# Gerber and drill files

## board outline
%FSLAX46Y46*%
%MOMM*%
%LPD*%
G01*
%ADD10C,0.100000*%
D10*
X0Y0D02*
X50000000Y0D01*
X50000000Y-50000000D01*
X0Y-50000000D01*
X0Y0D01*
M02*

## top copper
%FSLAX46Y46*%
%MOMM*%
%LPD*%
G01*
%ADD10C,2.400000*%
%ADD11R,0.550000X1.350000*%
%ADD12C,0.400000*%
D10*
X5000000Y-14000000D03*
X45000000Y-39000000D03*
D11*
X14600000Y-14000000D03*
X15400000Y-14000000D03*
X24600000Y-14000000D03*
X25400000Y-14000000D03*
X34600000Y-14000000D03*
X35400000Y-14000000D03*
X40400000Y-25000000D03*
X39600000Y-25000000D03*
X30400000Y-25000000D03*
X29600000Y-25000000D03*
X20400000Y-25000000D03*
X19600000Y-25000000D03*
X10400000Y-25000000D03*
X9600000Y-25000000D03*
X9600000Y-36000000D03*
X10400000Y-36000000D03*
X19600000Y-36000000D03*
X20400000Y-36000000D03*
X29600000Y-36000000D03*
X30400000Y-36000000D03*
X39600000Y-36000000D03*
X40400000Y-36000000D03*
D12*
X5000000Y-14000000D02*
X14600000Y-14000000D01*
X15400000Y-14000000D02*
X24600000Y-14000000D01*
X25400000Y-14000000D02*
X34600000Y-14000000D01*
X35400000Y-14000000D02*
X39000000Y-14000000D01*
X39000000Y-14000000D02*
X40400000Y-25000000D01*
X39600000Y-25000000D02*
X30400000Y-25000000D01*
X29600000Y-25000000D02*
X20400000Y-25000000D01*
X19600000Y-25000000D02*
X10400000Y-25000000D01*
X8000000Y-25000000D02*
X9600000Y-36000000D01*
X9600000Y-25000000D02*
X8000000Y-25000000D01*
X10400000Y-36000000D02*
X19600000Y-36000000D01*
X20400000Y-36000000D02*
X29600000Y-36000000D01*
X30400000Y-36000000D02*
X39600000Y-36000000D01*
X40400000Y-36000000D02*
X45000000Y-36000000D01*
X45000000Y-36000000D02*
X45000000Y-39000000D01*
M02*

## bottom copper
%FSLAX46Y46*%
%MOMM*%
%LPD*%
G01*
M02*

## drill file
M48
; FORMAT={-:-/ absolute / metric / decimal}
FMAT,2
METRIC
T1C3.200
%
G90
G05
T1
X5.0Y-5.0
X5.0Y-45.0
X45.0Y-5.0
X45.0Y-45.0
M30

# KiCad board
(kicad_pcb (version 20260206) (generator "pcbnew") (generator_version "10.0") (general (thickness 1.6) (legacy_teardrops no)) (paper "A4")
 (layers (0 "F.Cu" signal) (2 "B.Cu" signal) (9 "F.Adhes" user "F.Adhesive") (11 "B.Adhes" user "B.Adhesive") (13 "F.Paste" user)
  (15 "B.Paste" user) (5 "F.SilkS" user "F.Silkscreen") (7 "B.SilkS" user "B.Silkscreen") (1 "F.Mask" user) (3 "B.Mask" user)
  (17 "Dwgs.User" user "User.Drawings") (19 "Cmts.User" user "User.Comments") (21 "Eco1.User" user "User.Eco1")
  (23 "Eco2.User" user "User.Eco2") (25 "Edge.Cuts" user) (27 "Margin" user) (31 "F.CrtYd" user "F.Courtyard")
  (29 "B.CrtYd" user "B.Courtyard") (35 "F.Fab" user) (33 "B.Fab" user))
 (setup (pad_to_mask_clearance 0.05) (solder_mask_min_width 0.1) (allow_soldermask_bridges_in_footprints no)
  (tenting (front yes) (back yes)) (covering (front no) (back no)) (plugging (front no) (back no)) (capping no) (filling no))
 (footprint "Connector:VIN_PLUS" (layer "F.Cu") (at 5 14)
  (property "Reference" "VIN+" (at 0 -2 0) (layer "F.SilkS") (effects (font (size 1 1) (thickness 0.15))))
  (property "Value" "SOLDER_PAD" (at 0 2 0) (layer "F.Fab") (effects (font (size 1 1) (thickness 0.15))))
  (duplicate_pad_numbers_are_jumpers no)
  (pad "1" smd circle (at 0 0) (size 2.4 2.4) (layers "F.Cu" "F.Mask" "F.Paste") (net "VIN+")))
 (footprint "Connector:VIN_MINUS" (layer "F.Cu") (at 45 39)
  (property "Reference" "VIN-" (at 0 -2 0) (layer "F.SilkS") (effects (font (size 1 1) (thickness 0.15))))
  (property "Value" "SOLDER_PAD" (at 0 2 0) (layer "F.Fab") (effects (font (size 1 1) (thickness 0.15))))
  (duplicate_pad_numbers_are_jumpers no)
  (pad "1" smd circle (at 0 0) (size 2.4 2.4) (layers "F.Cu" "F.Mask" "F.Paste") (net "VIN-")))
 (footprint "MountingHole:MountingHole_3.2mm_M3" (layer "F.Cu") (at 5 5)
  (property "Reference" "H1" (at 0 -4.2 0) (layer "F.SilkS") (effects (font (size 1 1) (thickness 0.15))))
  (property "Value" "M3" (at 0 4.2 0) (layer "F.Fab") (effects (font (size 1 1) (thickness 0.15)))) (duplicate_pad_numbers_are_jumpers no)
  (pad "" np_thru_hole circle (at 0 0) (size 3.2 3.2) (drill 3.2) (layers "*.Cu" "*.Mask")))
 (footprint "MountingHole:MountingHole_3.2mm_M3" (layer "F.Cu") (at 45 5)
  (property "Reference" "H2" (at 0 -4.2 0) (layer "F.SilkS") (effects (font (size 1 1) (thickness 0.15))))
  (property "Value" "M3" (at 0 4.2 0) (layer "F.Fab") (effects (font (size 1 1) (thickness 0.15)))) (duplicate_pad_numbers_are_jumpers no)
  (pad "" np_thru_hole circle (at 0 0) (size 3.2 3.2) (drill 3.2) (layers "*.Cu" "*.Mask")))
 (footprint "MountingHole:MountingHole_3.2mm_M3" (layer "F.Cu") (at 5 45)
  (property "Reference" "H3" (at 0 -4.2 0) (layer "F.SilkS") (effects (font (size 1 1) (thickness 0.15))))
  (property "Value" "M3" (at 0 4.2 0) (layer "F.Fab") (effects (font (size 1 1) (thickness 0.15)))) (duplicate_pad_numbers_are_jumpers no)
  (pad "" np_thru_hole circle (at 0 0) (size 3.2 3.2) (drill 3.2) (layers "*.Cu" "*.Mask")))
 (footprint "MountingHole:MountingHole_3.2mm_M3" (layer "F.Cu") (at 45 45)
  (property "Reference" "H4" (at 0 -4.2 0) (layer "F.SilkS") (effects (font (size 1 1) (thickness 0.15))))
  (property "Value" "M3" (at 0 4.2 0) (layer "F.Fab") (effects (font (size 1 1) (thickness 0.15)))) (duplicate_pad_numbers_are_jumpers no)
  (pad "" np_thru_hole circle (at 0 0) (size 3.2 3.2) (drill 3.2) (layers "*.Cu" "*.Mask")))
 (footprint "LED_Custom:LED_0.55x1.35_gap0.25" (layer "F.Cu") (at 15 14)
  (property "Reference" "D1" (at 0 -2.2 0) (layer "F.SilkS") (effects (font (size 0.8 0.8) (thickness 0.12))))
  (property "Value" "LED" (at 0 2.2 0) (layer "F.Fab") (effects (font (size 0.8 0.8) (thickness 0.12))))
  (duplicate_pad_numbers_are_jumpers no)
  (pad "A" smd rect (at -0.4 0) (size 0.55 1.35) (layers "F.Cu" "F.Mask" "F.Paste") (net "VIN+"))
  (pad "K" smd rect (at 0.4 0) (size 0.55 1.35) (layers "F.Cu" "F.Mask" "F.Paste") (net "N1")))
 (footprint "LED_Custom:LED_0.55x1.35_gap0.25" (layer "F.Cu") (at 25 14)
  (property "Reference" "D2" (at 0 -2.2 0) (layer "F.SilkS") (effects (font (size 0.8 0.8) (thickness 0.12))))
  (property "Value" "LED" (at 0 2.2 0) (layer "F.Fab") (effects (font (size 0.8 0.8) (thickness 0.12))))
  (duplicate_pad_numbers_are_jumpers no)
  (pad "A" smd rect (at -0.4 0) (size 0.55 1.35) (layers "F.Cu" "F.Mask" "F.Paste") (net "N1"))
  (pad "K" smd rect (at 0.4 0) (size 0.55 1.35) (layers "F.Cu" "F.Mask" "F.Paste") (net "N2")))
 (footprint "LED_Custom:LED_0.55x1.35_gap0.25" (layer "F.Cu") (at 35 14)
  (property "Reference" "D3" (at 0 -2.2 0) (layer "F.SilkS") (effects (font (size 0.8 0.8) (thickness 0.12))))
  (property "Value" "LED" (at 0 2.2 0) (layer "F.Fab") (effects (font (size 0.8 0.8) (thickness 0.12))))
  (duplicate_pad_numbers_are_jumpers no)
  (pad "A" smd rect (at -0.4 0) (size 0.55 1.35) (layers "F.Cu" "F.Mask" "F.Paste") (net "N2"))
  (pad "K" smd rect (at 0.4 0) (size 0.55 1.35) (layers "F.Cu" "F.Mask" "F.Paste") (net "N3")))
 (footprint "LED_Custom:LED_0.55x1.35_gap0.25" (layer "F.Cu") (at 40 25 180)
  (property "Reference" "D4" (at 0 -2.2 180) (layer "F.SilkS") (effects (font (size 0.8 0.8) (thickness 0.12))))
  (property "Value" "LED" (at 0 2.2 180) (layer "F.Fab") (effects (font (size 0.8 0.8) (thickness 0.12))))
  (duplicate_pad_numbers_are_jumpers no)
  (pad "A" smd rect (at -0.4 0 180) (size 0.55 1.35) (layers "F.Cu" "F.Mask" "F.Paste") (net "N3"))
  (pad "K" smd rect (at 0.4 0 180) (size 0.55 1.35) (layers "F.Cu" "F.Mask" "F.Paste") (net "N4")))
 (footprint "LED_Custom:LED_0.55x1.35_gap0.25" (layer "F.Cu") (at 30 25 180)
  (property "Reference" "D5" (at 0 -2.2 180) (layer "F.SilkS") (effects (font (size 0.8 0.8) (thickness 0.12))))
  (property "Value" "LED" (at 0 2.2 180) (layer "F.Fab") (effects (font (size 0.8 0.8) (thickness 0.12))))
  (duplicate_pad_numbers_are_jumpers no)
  (pad "A" smd rect (at -0.4 0 180) (size 0.55 1.35) (layers "F.Cu" "F.Mask" "F.Paste") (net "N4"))
  (pad "K" smd rect (at 0.4 0 180) (size 0.55 1.35) (layers "F.Cu" "F.Mask" "F.Paste") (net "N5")))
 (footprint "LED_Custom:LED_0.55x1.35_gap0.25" (layer "F.Cu") (at 20 25 180)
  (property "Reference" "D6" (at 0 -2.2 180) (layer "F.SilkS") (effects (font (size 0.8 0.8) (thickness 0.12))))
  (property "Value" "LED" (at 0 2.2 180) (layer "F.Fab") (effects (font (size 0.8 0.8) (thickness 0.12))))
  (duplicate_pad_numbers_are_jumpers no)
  (pad "A" smd rect (at -0.4 0 180) (size 0.55 1.35) (layers "F.Cu" "F.Mask" "F.Paste") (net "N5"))
  (pad "K" smd rect (at 0.4 0 180) (size 0.55 1.35) (layers "F.Cu" "F.Mask" "F.Paste") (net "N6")))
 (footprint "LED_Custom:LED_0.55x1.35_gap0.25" (layer "F.Cu") (at 10 25 180)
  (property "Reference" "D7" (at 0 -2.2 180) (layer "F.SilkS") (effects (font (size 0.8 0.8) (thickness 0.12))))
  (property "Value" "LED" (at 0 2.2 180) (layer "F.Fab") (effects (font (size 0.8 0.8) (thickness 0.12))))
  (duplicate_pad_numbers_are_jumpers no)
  (pad "A" smd rect (at -0.4 0 180) (size 0.55 1.35) (layers "F.Cu" "F.Mask" "F.Paste") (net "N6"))
  (pad "K" smd rect (at 0.4 0 180) (size 0.55 1.35) (layers "F.Cu" "F.Mask" "F.Paste") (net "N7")))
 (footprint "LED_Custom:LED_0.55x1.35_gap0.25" (layer "F.Cu") (at 10 36)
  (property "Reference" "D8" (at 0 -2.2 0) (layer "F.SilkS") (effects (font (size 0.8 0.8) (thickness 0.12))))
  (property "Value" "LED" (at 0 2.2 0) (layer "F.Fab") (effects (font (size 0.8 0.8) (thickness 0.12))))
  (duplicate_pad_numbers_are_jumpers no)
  (pad "A" smd rect (at -0.4 0) (size 0.55 1.35) (layers "F.Cu" "F.Mask" "F.Paste") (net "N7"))
  (pad "K" smd rect (at 0.4 0) (size 0.55 1.35) (layers "F.Cu" "F.Mask" "F.Paste") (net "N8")))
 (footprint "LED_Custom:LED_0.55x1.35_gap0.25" (layer "F.Cu") (at 20 36)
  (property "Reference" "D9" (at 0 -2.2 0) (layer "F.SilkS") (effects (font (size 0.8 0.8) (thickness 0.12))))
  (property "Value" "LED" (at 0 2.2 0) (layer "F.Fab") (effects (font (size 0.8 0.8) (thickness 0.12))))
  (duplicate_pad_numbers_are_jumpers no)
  (pad "A" smd rect (at -0.4 0) (size 0.55 1.35) (layers "F.Cu" "F.Mask" "F.Paste") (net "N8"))
  (pad "K" smd rect (at 0.4 0) (size 0.55 1.35) (layers "F.Cu" "F.Mask" "F.Paste") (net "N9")))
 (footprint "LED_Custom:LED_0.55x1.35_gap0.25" (layer "F.Cu") (at 30 36)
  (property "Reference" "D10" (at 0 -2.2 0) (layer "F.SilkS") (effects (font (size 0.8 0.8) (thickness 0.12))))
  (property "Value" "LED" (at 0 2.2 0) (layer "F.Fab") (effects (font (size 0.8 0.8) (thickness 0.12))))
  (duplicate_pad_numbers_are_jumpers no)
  (pad "A" smd rect (at -0.4 0) (size 0.55 1.35) (layers "F.Cu" "F.Mask" "F.Paste") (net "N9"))
  (pad "K" smd rect (at 0.4 0) (size 0.55 1.35) (layers "F.Cu" "F.Mask" "F.Paste") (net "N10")))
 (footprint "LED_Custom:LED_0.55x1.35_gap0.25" (layer "F.Cu") (at 40 36)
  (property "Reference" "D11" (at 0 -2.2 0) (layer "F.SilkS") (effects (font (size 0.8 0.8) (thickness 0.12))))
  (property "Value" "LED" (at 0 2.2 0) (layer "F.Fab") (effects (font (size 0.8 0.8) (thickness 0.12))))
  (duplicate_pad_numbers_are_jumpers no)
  (pad "A" smd rect (at -0.4 0) (size 0.55 1.35) (layers "F.Cu" "F.Mask" "F.Paste") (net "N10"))
  (pad "K" smd rect (at 0.4 0) (size 0.55 1.35) (layers "F.Cu" "F.Mask" "F.Paste") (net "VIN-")))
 (gr_rect (start 0 0) (end 50 50) (stroke (width 0.1) (type solid)) (fill no) (layer "Edge.Cuts"))
 (segment (start 5 14) (end 14.6 14) (width 0.4) (layer "F.Cu") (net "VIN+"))
 (segment (start 40.4 36) (end 45 36) (width 0.4) (layer "F.Cu") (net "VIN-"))
 (segment (start 45 36) (end 45 39) (width 0.4) (layer "F.Cu") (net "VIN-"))
 (segment (start 15.4 14) (end 24.6 14) (width 0.4) (layer "F.Cu") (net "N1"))
 (segment (start 25.4 14) (end 34.6 14) (width 0.4) (layer "F.Cu") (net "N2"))
 (segment (start 35.4 14) (end 39 14) (width 0.4) (layer "F.Cu") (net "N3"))
 (segment (start 39 14) (end 40.4 25) (width 0.4) (layer "F.Cu") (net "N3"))
 (segment (start 39.6 25) (end 30.4 25) (width 0.4) (layer "F.Cu") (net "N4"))
 (segment (start 29.6 25) (end 20.4 25) (width 0.4) (layer "F.Cu") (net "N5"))
 (segment (start 19.6 25) (end 10.4 25) (width 0.4) (layer "F.Cu") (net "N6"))
 (segment (start 8 25) (end 9.6 36) (width 0.4) (layer "F.Cu") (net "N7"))
 (segment (start 9.6 25) (end 8 25) (width 0.4) (layer "F.Cu") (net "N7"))
 (segment (start 10.4 36) (end 19.6 36) (width 0.4) (layer "F.Cu") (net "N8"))
 (segment (start 20.4 36) (end 29.6 36) (width 0.4) (layer "F.Cu") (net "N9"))
 (segment (start 30.4 36) (end 39.6 36) (width 0.4) (layer "F.Cu") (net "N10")))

